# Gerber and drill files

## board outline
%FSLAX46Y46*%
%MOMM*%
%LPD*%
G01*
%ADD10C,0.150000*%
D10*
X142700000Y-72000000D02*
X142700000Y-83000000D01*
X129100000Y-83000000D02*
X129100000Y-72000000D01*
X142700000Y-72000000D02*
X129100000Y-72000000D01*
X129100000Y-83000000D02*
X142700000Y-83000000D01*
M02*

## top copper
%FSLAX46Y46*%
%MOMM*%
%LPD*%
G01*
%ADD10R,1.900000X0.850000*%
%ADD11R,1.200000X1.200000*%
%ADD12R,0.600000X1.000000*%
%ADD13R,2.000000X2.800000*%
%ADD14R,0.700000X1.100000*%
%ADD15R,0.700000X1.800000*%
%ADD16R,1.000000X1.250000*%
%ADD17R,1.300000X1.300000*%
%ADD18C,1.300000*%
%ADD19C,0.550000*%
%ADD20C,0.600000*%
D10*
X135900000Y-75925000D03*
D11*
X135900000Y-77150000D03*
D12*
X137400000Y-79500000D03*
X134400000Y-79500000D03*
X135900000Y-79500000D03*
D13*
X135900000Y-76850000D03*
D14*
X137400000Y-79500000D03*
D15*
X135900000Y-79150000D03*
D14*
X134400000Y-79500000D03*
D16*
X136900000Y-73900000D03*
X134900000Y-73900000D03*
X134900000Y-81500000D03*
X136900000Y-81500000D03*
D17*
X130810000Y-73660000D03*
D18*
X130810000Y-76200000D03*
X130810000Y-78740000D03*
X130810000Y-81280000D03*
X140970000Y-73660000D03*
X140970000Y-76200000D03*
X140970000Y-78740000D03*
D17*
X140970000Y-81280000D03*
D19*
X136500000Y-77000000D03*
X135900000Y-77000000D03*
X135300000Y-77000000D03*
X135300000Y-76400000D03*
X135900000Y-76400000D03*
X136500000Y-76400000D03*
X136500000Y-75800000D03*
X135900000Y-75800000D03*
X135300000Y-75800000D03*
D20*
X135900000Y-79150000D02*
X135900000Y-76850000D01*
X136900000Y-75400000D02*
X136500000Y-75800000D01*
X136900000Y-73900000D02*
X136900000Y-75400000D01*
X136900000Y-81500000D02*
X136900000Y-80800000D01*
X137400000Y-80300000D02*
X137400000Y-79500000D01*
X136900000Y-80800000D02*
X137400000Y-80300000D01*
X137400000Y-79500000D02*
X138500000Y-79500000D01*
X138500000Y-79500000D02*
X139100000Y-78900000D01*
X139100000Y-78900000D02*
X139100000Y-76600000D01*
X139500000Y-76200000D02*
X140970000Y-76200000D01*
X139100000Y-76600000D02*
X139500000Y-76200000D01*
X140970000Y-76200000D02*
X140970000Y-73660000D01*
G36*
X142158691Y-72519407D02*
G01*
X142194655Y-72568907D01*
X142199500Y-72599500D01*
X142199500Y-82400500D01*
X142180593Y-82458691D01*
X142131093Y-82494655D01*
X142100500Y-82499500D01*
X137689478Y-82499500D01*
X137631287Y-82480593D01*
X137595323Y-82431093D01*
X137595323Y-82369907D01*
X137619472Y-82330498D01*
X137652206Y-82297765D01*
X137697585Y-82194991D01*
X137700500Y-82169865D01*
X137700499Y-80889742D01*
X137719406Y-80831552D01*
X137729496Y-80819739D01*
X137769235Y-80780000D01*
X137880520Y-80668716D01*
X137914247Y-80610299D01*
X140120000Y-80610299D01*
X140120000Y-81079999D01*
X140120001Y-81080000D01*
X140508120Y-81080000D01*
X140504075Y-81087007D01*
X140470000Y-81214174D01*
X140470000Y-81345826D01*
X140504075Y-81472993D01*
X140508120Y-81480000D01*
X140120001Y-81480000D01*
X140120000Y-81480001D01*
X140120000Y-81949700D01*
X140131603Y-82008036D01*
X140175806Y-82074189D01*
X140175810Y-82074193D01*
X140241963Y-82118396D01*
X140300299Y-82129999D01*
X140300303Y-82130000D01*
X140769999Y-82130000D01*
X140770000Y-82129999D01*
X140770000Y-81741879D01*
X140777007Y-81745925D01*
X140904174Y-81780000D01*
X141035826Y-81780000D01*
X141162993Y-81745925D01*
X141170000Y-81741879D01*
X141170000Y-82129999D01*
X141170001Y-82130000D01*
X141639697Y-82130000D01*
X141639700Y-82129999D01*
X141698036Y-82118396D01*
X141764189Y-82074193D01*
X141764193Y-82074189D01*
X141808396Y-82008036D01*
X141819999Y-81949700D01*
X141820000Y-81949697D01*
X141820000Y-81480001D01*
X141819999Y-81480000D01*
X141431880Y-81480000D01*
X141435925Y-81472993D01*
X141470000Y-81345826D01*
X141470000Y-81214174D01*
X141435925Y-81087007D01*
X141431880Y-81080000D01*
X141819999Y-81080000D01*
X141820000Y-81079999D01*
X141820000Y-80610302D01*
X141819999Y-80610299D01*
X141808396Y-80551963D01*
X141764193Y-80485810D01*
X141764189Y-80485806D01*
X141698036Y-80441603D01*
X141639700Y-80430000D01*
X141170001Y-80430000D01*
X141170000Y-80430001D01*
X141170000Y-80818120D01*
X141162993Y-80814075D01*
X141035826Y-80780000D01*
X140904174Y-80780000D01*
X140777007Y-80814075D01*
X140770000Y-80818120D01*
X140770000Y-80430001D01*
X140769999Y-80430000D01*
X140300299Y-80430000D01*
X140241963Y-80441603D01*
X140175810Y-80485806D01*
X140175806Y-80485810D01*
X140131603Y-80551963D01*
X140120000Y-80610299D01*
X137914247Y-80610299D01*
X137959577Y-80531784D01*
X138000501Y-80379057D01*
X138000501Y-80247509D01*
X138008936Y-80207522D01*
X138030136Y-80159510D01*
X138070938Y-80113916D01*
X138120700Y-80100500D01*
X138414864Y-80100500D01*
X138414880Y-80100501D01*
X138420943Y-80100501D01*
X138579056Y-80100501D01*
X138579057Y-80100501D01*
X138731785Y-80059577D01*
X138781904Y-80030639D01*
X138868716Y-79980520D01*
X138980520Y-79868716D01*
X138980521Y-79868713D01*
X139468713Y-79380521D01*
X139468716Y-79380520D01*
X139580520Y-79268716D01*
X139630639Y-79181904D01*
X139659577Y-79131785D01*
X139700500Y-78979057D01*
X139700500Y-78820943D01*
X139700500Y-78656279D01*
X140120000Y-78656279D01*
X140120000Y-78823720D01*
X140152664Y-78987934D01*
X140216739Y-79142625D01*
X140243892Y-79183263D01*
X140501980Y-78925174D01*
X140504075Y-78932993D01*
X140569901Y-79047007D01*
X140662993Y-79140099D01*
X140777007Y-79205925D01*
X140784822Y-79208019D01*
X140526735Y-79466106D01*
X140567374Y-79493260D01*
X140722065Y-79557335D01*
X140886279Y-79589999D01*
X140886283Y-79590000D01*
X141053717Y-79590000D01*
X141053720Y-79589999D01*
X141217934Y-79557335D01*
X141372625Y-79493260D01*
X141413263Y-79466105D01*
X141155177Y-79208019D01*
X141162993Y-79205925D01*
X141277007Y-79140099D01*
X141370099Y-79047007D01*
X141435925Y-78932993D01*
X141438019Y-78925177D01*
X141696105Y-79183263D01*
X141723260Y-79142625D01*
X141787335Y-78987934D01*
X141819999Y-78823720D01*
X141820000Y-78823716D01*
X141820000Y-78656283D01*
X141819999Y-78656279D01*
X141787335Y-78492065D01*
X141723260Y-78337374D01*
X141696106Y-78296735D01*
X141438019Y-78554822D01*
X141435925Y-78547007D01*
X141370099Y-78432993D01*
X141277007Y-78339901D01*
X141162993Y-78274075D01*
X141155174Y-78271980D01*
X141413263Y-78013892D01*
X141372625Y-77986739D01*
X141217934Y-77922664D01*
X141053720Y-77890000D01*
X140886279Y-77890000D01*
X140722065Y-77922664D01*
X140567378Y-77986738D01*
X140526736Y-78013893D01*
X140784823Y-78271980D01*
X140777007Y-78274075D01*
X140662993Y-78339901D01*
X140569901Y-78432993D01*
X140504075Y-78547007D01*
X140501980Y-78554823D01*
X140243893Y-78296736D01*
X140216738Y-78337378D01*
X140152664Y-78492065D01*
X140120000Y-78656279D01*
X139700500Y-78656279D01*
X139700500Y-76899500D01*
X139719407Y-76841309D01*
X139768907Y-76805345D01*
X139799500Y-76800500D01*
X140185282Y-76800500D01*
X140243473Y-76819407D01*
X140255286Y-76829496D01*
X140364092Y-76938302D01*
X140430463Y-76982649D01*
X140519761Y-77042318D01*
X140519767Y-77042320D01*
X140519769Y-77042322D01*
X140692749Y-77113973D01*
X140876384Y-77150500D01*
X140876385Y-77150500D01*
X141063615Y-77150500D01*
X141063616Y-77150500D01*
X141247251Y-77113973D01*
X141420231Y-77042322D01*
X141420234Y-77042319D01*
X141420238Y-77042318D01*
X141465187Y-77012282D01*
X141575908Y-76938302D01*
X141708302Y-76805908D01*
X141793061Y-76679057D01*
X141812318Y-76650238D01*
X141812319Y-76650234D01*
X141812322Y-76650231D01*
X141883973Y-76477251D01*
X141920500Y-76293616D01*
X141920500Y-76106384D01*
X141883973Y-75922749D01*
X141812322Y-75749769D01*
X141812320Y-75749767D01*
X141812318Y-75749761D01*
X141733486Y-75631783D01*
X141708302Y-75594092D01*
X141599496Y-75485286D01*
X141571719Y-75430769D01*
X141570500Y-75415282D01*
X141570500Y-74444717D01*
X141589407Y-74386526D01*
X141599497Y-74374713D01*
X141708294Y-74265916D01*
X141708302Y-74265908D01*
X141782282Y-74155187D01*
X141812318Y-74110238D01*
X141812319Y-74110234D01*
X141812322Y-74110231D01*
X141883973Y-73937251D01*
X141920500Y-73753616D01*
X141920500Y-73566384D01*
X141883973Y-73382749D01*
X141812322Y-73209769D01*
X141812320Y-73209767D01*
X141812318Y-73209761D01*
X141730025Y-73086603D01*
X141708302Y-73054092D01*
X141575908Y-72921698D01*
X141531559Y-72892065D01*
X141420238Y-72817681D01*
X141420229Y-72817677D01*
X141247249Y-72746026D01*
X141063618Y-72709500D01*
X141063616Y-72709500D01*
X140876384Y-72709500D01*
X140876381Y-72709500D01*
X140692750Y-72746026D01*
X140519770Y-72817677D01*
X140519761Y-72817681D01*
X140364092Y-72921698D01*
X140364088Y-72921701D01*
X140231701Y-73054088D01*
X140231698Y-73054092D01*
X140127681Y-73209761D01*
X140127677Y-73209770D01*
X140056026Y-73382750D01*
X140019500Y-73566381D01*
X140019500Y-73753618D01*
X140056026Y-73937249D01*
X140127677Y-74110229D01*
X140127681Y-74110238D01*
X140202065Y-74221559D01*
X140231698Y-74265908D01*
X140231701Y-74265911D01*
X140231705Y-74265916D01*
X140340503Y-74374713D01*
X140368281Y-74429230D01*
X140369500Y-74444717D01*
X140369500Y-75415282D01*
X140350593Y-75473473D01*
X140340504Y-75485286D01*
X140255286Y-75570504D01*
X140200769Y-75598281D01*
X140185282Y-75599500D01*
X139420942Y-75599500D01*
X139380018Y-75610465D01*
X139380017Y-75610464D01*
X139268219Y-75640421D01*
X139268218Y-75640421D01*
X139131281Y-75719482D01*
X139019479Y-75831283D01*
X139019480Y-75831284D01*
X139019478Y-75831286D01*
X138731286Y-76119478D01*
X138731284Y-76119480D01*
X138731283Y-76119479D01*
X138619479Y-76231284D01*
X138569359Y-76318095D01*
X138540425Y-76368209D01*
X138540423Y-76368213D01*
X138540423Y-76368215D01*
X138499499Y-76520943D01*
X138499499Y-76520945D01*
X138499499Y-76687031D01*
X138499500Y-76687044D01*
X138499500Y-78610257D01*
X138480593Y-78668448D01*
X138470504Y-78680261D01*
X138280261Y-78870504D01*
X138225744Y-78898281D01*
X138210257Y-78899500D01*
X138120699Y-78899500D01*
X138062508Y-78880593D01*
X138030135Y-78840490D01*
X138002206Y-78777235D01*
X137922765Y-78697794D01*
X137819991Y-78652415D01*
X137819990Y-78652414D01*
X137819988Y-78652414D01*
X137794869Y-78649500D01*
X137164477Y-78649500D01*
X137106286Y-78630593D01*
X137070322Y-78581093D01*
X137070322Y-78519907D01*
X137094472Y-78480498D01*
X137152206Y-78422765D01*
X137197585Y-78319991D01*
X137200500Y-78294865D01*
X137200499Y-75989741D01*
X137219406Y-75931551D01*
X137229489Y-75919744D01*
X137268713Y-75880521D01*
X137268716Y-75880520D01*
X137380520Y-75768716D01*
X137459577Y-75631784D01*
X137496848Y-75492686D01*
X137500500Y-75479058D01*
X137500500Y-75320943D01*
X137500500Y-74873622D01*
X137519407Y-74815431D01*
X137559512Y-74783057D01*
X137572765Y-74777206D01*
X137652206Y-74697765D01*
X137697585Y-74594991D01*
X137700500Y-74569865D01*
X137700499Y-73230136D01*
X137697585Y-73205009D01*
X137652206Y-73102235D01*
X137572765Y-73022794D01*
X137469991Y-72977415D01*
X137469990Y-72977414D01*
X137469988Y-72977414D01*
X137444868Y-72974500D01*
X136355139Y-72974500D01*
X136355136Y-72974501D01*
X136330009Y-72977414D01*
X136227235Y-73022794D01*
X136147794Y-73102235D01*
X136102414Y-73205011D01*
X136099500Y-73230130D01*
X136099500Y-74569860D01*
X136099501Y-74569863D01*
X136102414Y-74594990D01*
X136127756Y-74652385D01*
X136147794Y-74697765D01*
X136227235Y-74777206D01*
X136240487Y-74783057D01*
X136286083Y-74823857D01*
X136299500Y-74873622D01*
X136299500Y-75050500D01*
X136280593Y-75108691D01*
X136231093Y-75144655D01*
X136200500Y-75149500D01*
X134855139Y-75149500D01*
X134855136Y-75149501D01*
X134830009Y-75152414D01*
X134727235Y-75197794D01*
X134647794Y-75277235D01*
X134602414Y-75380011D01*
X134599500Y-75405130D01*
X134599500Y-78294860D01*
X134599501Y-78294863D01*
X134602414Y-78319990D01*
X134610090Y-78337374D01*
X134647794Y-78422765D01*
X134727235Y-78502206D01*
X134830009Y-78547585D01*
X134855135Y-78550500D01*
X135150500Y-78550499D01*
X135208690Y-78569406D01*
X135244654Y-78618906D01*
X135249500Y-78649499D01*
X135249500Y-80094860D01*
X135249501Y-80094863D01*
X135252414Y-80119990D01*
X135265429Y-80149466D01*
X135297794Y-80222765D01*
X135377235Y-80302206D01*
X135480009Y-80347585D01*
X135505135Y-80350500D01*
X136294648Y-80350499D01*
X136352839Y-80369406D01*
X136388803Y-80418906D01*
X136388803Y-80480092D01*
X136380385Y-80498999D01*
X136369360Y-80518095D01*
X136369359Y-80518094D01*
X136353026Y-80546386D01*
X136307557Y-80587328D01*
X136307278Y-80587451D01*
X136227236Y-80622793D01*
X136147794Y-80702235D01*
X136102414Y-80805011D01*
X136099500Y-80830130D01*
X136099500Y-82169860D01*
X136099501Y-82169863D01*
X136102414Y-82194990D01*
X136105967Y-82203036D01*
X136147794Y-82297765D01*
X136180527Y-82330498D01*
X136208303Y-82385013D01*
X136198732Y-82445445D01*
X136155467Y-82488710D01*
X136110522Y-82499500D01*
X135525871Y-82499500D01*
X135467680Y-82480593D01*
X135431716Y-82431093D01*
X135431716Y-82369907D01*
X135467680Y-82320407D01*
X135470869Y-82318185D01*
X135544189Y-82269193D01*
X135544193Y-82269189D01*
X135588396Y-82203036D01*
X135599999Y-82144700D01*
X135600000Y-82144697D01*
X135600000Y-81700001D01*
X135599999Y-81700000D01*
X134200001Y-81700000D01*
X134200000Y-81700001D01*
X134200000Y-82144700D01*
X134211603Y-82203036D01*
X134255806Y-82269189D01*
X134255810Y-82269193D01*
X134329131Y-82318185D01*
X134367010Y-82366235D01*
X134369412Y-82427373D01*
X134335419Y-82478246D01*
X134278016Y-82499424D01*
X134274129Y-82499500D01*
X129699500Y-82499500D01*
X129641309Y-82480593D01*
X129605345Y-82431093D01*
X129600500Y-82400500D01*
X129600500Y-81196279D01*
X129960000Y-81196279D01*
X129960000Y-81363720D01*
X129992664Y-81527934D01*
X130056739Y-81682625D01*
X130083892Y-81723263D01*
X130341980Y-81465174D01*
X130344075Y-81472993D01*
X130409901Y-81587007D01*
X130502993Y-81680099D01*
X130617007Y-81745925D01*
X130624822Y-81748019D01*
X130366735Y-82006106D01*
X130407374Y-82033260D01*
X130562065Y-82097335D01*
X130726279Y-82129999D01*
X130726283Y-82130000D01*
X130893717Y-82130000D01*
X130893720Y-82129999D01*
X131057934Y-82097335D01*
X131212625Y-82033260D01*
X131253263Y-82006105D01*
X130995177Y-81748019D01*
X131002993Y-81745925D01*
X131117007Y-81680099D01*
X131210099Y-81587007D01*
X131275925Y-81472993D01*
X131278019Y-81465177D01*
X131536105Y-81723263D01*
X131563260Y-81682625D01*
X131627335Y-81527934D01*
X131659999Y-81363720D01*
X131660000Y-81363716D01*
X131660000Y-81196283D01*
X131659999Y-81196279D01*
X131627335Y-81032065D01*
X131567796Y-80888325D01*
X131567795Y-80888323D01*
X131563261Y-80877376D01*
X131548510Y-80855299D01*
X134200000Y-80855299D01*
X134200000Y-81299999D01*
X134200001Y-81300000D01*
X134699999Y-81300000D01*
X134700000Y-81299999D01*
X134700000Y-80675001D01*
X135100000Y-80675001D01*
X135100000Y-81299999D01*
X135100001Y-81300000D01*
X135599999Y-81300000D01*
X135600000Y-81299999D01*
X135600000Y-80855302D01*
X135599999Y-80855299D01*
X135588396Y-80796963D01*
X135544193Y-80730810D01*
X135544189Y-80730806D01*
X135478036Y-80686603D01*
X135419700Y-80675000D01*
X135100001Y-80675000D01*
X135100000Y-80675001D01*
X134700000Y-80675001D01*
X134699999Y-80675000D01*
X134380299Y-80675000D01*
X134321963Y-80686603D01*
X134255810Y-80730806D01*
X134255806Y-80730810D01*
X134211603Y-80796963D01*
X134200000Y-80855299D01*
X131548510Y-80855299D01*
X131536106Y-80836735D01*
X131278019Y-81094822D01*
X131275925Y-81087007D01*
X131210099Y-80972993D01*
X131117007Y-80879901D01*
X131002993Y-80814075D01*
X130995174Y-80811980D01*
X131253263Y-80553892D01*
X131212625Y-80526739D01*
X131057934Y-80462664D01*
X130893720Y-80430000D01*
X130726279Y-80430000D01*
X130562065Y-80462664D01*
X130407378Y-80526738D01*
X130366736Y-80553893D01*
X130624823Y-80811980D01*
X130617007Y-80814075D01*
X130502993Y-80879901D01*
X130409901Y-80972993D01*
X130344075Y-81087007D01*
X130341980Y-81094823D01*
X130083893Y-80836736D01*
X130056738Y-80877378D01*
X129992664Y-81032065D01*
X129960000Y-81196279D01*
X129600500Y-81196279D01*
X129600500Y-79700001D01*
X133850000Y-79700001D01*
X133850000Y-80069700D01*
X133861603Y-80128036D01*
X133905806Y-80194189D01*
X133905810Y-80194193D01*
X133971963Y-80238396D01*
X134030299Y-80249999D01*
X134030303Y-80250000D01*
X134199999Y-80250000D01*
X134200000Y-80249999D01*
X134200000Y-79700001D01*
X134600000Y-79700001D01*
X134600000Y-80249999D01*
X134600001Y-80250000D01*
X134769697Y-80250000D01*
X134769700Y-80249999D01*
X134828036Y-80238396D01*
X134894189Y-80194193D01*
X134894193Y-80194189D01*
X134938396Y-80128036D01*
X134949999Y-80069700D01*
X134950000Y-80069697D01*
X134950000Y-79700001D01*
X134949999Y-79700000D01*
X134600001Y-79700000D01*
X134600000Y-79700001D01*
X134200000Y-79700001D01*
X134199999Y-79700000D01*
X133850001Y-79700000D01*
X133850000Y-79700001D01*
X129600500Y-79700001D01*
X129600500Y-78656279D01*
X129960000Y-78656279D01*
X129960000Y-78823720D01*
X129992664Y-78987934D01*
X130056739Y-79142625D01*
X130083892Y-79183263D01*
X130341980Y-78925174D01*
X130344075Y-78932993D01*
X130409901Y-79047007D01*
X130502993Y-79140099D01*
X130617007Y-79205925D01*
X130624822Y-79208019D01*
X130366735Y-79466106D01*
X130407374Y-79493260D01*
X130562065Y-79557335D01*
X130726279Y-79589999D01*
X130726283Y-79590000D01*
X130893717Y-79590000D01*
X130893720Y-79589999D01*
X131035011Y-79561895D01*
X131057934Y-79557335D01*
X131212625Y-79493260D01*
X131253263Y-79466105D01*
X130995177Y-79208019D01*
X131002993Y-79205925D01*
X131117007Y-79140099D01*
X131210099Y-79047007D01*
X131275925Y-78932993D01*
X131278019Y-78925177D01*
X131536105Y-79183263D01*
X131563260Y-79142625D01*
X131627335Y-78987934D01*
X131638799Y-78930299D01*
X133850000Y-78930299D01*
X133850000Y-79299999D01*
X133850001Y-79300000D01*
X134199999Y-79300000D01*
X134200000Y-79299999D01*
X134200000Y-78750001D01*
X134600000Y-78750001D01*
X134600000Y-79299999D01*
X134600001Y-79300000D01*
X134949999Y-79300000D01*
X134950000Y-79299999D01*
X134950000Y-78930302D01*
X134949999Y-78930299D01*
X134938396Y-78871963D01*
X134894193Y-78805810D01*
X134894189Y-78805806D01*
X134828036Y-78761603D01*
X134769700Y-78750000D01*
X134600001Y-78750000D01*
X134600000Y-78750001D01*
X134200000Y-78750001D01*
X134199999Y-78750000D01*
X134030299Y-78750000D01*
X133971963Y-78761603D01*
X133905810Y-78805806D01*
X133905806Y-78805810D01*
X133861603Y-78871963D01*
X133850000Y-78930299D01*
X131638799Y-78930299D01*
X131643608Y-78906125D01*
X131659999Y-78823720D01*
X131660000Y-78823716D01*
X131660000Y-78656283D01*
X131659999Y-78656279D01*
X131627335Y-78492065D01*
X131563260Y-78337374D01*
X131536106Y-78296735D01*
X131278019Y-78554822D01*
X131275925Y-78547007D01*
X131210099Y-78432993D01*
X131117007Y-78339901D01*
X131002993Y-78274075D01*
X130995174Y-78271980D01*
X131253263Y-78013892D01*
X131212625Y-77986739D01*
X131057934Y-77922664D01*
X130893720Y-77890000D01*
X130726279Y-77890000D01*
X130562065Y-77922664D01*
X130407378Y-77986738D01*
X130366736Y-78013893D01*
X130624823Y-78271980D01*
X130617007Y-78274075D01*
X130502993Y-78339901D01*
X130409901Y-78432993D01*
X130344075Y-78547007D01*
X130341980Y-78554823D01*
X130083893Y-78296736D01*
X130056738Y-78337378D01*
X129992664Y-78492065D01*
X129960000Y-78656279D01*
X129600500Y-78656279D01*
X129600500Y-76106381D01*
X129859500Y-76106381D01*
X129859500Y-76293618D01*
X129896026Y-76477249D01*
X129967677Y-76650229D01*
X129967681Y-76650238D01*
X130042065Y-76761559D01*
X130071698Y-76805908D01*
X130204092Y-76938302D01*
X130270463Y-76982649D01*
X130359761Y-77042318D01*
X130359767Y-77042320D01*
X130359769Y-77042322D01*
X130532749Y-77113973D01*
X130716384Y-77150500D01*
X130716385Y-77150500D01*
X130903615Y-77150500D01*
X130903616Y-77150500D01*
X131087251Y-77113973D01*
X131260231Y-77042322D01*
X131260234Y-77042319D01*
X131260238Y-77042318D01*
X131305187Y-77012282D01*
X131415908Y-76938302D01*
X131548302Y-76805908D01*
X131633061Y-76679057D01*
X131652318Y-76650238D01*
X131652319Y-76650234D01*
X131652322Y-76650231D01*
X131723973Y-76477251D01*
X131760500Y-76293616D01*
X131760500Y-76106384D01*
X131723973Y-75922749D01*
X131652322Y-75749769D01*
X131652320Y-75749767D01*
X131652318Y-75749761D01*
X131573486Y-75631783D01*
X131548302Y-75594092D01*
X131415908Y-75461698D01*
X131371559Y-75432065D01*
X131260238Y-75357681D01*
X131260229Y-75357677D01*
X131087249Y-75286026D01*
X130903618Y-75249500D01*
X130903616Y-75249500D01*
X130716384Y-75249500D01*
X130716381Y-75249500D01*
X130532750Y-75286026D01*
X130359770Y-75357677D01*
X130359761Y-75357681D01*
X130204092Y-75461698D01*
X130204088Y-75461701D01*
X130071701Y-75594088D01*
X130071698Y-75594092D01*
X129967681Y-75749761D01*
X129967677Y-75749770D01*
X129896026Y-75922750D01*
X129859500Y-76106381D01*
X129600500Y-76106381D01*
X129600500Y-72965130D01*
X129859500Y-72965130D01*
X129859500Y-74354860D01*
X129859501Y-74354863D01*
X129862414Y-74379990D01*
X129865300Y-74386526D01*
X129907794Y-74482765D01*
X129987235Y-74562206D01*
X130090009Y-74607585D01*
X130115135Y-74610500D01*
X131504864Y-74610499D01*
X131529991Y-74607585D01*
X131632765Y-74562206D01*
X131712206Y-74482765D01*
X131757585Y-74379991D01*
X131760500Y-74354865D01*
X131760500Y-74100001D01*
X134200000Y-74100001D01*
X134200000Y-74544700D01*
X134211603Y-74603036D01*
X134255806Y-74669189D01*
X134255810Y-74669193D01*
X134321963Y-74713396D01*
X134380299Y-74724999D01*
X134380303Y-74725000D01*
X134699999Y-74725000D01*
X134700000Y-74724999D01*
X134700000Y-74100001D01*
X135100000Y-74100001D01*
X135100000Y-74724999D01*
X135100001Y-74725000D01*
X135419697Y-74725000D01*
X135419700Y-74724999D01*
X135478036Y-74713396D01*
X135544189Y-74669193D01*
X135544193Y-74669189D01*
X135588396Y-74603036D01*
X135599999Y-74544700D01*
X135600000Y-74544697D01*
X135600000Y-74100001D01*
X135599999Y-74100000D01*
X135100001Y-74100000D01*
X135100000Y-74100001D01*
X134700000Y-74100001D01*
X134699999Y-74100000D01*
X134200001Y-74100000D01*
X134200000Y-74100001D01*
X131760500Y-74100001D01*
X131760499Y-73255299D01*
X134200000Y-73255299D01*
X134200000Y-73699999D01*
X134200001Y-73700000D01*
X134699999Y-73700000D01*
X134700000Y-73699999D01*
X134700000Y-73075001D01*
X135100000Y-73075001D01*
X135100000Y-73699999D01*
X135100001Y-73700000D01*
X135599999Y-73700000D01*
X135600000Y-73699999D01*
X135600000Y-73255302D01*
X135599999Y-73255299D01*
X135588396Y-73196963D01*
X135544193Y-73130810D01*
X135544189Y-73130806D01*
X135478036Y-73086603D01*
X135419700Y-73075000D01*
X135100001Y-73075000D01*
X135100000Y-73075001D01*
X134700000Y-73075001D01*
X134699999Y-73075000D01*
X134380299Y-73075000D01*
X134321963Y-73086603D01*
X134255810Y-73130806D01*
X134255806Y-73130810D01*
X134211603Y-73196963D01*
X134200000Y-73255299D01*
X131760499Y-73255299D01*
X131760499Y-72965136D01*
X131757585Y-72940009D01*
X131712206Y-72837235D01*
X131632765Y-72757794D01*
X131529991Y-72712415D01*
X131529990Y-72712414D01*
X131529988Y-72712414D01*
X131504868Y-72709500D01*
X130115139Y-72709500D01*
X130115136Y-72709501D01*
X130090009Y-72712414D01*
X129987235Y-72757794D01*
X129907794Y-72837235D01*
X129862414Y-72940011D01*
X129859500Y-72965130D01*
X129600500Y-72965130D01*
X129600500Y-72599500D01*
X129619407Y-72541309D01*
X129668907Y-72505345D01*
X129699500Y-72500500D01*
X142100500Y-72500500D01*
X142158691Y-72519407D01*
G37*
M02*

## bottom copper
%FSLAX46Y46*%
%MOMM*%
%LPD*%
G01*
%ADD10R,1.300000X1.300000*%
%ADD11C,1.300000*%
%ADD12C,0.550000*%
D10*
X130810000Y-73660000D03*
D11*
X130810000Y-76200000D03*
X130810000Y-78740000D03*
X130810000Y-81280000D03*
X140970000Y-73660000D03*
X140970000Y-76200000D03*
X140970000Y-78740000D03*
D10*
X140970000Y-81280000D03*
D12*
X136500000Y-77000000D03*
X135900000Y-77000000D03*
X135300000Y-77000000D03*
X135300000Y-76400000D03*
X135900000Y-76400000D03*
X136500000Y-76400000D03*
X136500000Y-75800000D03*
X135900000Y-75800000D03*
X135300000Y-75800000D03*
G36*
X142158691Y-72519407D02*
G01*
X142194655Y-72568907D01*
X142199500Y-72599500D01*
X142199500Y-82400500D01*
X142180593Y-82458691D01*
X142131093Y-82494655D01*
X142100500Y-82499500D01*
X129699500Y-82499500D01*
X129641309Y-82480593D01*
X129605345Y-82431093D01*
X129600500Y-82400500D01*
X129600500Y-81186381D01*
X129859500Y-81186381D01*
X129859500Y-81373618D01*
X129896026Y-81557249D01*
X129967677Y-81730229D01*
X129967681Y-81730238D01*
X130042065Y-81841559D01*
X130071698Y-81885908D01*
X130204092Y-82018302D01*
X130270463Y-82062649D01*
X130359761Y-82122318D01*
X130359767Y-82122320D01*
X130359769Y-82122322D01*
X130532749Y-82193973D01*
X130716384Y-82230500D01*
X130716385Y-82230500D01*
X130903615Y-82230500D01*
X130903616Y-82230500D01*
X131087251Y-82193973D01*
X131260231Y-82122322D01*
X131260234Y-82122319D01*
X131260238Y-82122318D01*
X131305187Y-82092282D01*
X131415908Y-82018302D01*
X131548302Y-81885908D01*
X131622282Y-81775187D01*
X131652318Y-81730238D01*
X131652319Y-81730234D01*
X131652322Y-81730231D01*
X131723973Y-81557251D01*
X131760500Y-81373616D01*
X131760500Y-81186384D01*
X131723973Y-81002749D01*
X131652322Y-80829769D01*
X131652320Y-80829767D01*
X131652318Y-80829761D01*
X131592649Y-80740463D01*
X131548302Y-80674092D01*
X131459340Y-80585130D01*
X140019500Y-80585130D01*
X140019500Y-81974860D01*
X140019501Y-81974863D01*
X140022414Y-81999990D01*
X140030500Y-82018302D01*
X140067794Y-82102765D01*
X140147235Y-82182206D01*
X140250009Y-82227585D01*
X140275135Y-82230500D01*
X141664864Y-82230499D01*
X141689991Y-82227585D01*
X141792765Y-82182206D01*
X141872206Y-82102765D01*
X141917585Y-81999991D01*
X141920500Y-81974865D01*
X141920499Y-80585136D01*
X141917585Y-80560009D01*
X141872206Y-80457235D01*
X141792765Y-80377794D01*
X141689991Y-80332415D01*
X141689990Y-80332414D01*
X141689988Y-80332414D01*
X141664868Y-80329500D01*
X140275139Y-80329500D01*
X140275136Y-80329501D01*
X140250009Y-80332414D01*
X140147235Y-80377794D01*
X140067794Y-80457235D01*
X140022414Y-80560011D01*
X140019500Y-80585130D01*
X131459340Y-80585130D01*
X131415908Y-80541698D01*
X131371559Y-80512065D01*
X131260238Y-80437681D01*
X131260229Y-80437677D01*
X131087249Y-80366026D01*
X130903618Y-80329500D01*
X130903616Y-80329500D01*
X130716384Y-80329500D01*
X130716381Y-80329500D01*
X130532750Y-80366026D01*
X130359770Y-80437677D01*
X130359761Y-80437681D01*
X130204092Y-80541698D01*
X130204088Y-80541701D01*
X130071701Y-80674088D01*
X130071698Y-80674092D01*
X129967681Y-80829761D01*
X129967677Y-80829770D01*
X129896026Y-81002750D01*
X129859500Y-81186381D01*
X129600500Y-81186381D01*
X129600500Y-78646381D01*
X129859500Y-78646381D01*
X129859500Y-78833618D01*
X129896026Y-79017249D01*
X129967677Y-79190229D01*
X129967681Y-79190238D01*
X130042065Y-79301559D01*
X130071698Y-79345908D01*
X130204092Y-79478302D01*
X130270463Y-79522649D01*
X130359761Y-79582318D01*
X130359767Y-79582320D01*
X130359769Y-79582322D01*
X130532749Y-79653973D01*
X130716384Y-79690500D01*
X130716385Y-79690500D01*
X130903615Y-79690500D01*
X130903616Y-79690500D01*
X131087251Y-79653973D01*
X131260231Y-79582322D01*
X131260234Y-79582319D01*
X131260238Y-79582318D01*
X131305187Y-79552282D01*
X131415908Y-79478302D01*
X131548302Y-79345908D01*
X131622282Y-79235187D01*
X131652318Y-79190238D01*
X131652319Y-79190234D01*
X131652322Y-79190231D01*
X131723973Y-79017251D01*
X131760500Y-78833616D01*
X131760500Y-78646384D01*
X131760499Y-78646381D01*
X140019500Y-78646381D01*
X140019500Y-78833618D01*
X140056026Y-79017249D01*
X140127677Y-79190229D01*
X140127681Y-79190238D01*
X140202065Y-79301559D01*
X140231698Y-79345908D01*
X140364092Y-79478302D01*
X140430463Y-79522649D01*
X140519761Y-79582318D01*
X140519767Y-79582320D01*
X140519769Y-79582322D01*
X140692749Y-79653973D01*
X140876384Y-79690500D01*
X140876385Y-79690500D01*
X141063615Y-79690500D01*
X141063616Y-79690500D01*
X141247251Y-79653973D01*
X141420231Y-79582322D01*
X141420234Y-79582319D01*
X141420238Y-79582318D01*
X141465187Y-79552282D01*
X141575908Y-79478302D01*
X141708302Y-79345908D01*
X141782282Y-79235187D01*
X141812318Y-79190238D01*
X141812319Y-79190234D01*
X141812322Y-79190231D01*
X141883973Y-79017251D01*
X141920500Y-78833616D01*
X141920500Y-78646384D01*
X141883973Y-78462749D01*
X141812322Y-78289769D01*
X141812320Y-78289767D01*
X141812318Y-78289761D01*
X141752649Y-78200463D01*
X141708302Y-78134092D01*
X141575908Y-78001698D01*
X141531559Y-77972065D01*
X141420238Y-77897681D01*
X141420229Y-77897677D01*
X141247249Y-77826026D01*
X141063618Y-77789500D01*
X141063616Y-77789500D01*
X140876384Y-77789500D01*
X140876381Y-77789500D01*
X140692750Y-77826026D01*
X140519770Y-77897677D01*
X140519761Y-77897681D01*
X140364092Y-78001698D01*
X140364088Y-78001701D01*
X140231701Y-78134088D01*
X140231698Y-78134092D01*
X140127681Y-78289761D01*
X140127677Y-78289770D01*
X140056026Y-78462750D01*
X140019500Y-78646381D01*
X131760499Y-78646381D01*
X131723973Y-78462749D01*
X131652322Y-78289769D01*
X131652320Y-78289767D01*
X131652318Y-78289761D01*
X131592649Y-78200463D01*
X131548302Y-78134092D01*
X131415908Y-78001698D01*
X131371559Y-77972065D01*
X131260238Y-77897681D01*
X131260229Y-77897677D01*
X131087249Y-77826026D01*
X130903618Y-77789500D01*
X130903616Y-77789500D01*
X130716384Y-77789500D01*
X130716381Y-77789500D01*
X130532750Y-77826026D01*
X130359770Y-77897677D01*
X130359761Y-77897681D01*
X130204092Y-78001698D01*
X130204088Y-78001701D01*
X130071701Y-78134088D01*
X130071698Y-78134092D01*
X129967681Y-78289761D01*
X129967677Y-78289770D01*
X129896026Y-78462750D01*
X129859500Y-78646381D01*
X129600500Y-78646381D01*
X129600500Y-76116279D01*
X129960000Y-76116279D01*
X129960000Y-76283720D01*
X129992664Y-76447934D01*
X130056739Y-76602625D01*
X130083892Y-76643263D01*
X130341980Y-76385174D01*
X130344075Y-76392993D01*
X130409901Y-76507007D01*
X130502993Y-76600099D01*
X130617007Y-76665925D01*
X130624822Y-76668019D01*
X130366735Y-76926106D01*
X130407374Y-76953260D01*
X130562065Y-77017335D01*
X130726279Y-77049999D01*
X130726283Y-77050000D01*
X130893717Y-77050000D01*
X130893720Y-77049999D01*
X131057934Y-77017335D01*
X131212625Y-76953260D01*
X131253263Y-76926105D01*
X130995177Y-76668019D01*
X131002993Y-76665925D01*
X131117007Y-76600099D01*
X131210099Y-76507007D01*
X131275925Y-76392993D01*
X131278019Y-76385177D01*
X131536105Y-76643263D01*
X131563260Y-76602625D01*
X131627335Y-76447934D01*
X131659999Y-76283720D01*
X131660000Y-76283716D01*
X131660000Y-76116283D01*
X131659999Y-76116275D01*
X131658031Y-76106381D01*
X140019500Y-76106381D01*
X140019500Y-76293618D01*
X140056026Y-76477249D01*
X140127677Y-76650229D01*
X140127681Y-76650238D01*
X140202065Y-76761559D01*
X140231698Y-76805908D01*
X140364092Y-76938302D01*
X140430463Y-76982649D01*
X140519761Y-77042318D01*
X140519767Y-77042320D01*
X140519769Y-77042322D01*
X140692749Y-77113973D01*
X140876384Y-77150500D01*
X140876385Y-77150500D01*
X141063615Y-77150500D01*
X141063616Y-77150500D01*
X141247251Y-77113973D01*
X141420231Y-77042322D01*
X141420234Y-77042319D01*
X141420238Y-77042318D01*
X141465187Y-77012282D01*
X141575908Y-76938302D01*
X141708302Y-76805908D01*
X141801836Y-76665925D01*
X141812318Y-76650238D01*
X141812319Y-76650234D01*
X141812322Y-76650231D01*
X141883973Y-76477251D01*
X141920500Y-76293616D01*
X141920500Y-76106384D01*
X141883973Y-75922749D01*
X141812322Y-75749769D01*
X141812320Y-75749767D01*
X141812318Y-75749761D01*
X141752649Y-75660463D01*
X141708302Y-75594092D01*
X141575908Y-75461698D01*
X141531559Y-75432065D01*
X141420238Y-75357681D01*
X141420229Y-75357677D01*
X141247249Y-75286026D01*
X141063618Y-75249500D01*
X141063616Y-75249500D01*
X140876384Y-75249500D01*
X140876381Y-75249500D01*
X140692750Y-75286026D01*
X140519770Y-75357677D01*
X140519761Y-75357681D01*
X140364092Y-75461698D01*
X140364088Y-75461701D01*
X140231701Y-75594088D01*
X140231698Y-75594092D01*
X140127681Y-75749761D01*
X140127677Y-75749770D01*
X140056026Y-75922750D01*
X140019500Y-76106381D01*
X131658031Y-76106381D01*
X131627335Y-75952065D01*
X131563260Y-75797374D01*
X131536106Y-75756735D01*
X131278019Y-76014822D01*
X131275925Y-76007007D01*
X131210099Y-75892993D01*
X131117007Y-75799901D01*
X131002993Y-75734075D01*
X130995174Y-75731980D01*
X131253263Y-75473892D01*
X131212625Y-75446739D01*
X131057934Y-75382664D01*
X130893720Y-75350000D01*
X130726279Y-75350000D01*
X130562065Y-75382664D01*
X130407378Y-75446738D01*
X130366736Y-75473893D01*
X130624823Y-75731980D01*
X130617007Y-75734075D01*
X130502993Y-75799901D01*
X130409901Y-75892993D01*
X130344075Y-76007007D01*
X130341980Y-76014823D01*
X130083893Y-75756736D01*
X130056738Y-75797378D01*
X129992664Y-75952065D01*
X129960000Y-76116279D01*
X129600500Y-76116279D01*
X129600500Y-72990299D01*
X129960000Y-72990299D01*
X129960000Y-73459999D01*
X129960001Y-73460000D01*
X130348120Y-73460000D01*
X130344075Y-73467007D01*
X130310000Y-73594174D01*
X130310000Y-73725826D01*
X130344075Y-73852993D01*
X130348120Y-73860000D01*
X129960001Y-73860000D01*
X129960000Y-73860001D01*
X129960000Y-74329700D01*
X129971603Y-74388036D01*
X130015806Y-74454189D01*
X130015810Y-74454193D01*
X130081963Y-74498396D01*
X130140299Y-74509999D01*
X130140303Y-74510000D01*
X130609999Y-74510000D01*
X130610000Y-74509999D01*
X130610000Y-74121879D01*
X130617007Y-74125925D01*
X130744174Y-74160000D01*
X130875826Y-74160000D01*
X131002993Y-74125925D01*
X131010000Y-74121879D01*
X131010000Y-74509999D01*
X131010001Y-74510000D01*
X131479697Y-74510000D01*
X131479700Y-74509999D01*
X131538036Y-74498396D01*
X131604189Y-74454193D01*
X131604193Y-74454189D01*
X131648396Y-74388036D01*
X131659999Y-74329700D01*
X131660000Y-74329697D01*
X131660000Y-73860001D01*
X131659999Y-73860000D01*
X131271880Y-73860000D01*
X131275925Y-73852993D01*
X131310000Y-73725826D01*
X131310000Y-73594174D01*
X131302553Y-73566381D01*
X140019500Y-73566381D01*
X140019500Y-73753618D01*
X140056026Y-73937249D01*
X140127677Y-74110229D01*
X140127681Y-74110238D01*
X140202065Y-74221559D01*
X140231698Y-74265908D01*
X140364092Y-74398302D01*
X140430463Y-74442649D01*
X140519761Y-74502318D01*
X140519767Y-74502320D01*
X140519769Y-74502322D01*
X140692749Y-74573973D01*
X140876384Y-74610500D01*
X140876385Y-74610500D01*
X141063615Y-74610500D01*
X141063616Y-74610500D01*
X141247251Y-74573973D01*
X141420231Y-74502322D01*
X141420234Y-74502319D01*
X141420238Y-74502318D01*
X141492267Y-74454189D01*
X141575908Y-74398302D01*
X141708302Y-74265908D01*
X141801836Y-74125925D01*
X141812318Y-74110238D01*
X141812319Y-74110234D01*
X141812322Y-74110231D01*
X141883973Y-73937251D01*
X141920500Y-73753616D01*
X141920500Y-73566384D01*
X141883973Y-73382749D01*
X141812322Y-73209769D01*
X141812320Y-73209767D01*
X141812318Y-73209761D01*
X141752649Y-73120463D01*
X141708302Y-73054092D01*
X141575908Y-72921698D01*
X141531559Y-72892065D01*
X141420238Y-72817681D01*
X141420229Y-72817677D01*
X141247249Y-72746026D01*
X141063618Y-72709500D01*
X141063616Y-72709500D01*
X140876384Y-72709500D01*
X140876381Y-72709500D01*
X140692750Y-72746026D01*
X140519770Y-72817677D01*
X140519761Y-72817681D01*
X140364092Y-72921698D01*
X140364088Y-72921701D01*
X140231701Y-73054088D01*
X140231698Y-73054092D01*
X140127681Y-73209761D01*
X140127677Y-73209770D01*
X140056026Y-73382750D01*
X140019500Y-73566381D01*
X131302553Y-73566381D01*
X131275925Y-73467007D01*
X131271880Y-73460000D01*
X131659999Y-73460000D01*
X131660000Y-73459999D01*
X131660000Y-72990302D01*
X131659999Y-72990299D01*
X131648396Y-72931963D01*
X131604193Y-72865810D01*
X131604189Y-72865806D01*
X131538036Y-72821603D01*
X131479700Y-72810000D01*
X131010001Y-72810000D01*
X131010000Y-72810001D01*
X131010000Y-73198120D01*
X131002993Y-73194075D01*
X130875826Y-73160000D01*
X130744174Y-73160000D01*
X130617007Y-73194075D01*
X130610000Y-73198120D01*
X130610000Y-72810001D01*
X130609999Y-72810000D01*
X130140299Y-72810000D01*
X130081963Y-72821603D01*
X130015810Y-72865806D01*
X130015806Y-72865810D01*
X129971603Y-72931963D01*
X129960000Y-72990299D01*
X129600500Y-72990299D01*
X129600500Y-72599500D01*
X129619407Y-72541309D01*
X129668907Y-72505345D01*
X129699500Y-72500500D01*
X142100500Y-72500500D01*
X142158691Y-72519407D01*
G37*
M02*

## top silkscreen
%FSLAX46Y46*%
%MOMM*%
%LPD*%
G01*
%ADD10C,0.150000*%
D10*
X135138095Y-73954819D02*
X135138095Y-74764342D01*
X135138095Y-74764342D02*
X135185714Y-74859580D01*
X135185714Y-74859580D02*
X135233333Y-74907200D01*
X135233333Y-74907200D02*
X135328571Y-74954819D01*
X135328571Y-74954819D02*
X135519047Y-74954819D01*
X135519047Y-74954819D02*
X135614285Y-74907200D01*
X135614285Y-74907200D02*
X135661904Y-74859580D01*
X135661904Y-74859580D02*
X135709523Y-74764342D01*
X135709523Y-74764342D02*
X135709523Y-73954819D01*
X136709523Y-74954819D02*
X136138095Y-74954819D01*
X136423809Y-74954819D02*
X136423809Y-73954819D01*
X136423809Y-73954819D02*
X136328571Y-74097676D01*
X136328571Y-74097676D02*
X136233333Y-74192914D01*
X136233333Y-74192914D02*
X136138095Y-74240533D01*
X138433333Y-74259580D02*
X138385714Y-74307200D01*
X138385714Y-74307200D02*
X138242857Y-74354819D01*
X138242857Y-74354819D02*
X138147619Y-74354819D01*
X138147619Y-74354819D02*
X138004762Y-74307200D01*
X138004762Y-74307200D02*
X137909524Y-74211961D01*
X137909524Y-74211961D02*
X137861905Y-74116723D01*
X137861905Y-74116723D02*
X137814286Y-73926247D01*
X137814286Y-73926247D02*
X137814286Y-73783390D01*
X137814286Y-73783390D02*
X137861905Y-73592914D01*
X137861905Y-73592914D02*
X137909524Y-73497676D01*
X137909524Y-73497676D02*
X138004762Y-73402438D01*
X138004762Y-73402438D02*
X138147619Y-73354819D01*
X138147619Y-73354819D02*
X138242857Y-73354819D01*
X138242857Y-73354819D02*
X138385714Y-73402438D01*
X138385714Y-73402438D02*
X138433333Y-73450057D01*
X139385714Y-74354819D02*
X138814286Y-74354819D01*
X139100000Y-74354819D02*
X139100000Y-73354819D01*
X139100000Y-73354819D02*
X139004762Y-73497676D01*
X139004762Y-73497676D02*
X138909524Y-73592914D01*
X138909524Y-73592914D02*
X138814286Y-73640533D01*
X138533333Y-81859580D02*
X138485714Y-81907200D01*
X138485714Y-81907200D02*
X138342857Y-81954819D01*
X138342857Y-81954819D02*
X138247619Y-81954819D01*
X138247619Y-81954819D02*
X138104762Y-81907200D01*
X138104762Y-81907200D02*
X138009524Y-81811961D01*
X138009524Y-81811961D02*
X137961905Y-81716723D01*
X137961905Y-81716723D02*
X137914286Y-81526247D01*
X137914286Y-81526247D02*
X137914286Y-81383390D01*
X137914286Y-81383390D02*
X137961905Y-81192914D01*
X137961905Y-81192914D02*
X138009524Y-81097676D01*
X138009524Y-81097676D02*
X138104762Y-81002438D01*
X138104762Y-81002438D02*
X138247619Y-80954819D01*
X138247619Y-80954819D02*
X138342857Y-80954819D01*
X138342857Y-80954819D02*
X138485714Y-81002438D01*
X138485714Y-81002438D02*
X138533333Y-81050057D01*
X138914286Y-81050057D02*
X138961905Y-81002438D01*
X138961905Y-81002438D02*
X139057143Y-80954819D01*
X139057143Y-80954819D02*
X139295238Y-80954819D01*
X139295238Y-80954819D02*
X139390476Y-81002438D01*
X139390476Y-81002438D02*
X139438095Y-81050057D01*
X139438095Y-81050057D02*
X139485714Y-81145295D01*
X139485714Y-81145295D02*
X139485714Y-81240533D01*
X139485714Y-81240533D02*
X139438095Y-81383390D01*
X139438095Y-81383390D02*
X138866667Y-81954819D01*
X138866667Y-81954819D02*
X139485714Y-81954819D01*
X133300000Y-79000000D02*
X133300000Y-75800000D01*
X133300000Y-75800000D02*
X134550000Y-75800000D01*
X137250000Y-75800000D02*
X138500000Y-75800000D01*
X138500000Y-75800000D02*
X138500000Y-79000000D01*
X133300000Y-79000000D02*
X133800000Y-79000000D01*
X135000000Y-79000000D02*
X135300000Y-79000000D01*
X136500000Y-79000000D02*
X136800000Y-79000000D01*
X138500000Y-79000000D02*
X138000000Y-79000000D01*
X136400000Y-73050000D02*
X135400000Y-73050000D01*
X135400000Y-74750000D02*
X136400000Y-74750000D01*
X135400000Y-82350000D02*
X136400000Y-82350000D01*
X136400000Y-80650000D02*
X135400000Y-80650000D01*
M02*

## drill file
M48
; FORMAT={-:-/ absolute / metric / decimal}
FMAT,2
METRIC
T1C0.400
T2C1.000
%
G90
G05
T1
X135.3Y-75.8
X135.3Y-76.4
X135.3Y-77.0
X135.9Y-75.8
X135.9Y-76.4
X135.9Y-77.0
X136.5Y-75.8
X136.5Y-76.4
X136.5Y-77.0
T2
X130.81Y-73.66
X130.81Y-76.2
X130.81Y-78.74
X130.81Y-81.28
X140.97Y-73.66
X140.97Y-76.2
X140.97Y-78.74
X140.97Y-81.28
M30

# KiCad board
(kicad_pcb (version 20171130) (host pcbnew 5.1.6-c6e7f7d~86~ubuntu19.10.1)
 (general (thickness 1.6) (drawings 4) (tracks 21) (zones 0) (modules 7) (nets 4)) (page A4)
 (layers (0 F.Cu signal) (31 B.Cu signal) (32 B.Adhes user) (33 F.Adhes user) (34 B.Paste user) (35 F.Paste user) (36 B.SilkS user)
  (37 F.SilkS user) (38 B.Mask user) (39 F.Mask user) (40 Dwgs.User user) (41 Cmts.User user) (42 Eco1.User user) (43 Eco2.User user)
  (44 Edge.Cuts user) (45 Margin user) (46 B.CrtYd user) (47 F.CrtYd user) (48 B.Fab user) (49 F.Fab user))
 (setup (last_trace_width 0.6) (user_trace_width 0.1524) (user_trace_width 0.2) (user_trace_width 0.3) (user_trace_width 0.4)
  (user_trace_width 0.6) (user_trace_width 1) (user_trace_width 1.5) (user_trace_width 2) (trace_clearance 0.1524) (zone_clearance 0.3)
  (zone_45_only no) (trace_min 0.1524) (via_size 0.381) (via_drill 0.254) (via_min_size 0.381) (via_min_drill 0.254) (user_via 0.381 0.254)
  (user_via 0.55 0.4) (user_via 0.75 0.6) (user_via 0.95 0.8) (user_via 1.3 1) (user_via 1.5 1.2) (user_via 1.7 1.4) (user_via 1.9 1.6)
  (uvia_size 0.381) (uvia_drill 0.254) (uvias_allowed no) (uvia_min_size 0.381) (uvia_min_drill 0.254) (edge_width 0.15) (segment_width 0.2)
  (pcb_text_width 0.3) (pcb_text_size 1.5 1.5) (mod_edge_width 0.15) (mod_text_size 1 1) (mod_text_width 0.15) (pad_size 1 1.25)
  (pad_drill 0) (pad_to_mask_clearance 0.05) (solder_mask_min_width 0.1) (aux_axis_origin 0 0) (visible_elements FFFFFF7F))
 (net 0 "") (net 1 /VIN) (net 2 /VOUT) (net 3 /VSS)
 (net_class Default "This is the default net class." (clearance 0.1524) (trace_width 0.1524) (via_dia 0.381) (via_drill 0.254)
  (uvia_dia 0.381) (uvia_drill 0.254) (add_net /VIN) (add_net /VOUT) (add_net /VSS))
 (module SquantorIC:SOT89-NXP (layer F.Cu) (at 135.9 77.75)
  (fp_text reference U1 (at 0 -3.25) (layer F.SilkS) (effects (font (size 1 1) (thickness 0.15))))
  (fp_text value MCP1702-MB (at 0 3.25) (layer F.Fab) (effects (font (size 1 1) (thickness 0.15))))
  (fp_line (start -2.6 1.25) (end -2.6 -1.95) (layer F.SilkS) (width 0.15))
  (fp_line (start -2.6 -1.95) (end -1.35 -1.95) (layer F.SilkS) (width 0.15))
  (fp_line (start 1.35 -1.95) (end 2.6 -1.95) (layer F.SilkS) (width 0.15))
  (fp_line (start 2.6 -1.95) (end 2.6 1.25) (layer F.SilkS) (width 0.15))
  (fp_line (start -2.6 1.25) (end -2.1 1.25) (layer F.SilkS) (width 0.15))
  (fp_line (start -0.9 1.25) (end -0.6 1.25) (layer F.SilkS) (width 0.15))
  (fp_line (start 0.6 1.25) (end 0.9 1.25) (layer F.SilkS) (width 0.15))
  (fp_line (start 2.6 1.25) (end 2.1 1.25) (layer F.SilkS) (width 0.15))
  (pad 2 smd rect (at 0 -1.825) (size 1.9 0.85) (layers F.Cu F.Paste) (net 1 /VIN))
  (pad 2 smd rect (at 0 -0.6) (size 1.2 1.2) (layers F.Cu F.Paste) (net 1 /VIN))
  (pad 3 smd rect (at 1.5 1.75) (size 0.6 1) (layers F.Cu F.Paste) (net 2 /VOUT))
  (pad 1 smd rect (at -1.5 1.75) (size 0.6 1) (layers F.Cu F.Paste) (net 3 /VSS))
  (pad 2 smd rect (at 0 1.75) (size 0.6 1) (layers F.Cu F.Paste) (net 1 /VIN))
  (pad 2 smd rect (at 0 -0.9) (size 2 2.8) (layers F.Cu F.Mask) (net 1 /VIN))
  (pad 3 smd rect (at 1.5 1.75) (size 0.7 1.1) (layers F.Cu F.Mask) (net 2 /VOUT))
  (pad 2 smd rect (at 0 1.4) (size 0.7 1.8) (layers F.Cu F.Mask) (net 1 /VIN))
  (pad 1 smd rect (at -1.5 1.75) (size 0.7 1.1) (layers F.Cu F.Mask) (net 3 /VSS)))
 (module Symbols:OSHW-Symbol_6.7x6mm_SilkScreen (layer B.Cu) (at 135.9 75.3 180)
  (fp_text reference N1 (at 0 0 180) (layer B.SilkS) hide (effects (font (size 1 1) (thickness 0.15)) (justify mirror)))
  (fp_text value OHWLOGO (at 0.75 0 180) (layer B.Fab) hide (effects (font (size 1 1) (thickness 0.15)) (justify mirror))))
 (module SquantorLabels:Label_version (layer B.Cu) (at 135.3 80.01 90)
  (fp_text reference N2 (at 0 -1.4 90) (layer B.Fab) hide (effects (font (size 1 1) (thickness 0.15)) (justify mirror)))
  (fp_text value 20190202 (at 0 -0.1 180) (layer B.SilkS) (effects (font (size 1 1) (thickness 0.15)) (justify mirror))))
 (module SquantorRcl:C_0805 (layer F.Cu) (at 135.9 73.9 180)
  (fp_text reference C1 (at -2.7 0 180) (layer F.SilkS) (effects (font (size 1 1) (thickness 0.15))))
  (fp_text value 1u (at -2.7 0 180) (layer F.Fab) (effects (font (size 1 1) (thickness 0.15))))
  (fp_line (start -0.5 0.85) (end 0.5 0.85) (layer F.SilkS) (width 0.15))
  (fp_line (start 0.5 -0.85) (end -0.5 -0.85) (layer F.SilkS) (width 0.15))
  (pad 1 smd rect (at -1 0 180) (size 1 1.25) (layers F.Cu F.Paste F.Mask) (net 1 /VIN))
  (pad 2 smd rect (at 1 0 180) (size 1 1.25) (layers F.Cu F.Paste F.Mask) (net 3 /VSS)))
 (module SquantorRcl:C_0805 (layer F.Cu) (at 135.9 81.5 180)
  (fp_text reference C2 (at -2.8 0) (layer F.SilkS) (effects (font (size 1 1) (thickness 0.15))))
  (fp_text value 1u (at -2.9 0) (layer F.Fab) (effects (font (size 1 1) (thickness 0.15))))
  (fp_line (start 0.5 -0.85) (end -0.5 -0.85) (layer F.SilkS) (width 0.15))
  (fp_line (start -0.5 0.85) (end 0.5 0.85) (layer F.SilkS) (width 0.15))
  (pad 2 smd rect (at 1 0 180) (size 1 1.25) (layers F.Cu F.Paste F.Mask) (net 3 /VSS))
  (pad 1 smd rect (at -1 0 180) (size 1 1.25) (layers F.Cu F.Paste F.Mask) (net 2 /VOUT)))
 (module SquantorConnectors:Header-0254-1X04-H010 (layer B.Cu) (at 130.81 77.47 270)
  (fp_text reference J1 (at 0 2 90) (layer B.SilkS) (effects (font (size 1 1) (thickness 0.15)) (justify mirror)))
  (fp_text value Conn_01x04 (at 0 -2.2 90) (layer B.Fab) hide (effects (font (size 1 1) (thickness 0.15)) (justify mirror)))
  (pad 1 thru_hole rect (at -3.81 0 90) (size 1.3 1.3) (drill 1) (layers *.Cu *.Mask) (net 1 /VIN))
  (pad 2 thru_hole circle (at -1.27 0 90) (size 1.3 1.3) (drill 1) (layers *.Cu *.Mask) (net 1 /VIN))
  (pad 3 thru_hole circle (at 1.27 0 90) (size 1.3 1.3) (drill 1) (layers *.Cu *.Mask) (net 3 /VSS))
  (pad 4 thru_hole circle (at 3.81 0 90) (size 1.3 1.3) (drill 1) (layers *.Cu *.Mask) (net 3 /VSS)))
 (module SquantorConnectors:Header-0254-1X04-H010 (layer B.Cu) (at 140.97 77.47 90)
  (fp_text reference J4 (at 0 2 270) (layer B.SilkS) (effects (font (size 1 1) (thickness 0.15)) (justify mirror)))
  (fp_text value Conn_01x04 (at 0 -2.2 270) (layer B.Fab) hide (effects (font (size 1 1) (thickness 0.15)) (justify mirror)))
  (pad 4 thru_hole circle (at 3.81 0 270) (size 1.3 1.3) (drill 1) (layers *.Cu *.Mask) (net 2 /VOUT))
  (pad 3 thru_hole circle (at 1.27 0 270) (size 1.3 1.3) (drill 1) (layers *.Cu *.Mask) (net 2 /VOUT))
  (pad 2 thru_hole circle (at -1.27 0 270) (size 1.3 1.3) (drill 1) (layers *.Cu *.Mask) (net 3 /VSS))
  (pad 1 thru_hole rect (at -3.81 0 270) (size 1.3 1.3) (drill 1) (layers *.Cu *.Mask) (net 3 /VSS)))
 (gr_line (start 142.7 72) (end 142.7 83) (layer Edge.Cuts) (width 0.15))
 (gr_line (start 129.1 83) (end 129.1 72) (layer Edge.Cuts) (width 0.15))
 (gr_line (start 142.7 72) (end 129.1 72) (layer Edge.Cuts) (width 0.15))
 (gr_line (start 129.1 83) (end 142.7 83) (layer Edge.Cuts) (width 0.15))
 (via (at 136.5 77) (size 0.55) (drill 0.4) (layers F.Cu B.Cu) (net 1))
 (via (at 135.9 77) (size 0.55) (drill 0.4) (layers F.Cu B.Cu) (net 1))
 (via (at 135.3 77) (size 0.55) (drill 0.4) (layers F.Cu B.Cu) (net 1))
 (via (at 135.3 76.4) (size 0.55) (drill 0.4) (layers F.Cu B.Cu) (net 1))
 (via (at 135.9 76.4) (size 0.55) (drill 0.4) (layers F.Cu B.Cu) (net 1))
 (via (at 136.5 76.4) (size 0.55) (drill 0.4) (layers F.Cu B.Cu) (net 1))
 (via (at 136.5 75.8) (size 0.55) (drill 0.4) (layers F.Cu B.Cu) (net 1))
 (via (at 135.9 75.8) (size 0.55) (drill 0.4) (layers F.Cu B.Cu) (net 1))
 (via (at 135.3 75.8) (size 0.55) (drill 0.4) (layers F.Cu B.Cu) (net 1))
 (segment (start 135.9 79.15) (end 135.9 76.85) (width 0.6) (layer F.Cu) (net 1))
 (segment (start 136.9 75.4) (end 136.5 75.8) (width 0.6) (layer F.Cu) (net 1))
 (segment (start 136.9 73.9) (end 136.9 75.4) (width 0.6) (layer F.Cu) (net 1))
 (segment (start 136.9 81.5) (end 136.9 80.8) (width 0.6) (layer F.Cu) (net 2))
 (segment (start 137.4 80.3) (end 137.4 79.5) (width 0.6) (layer F.Cu) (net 2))
 (segment (start 136.9 80.8) (end 137.4 80.3) (width 0.6) (layer F.Cu) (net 2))
 (segment (start 137.4 79.5) (end 138.5 79.5) (width 0.6) (layer F.Cu) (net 2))
 (segment (start 138.5 79.5) (end 139.1 78.9) (width 0.6) (layer F.Cu) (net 2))
 (segment (start 139.1 78.9) (end 139.1 76.6) (width 0.6) (layer F.Cu) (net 2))
 (segment (start 139.5 76.2) (end 140.97 76.2) (width 0.6) (layer F.Cu) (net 2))
 (segment (start 139.1 76.6) (end 139.5 76.2) (width 0.6) (layer F.Cu) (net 2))
 (segment (start 140.97 76.2) (end 140.97 73.66) (width 0.6) (layer F.Cu) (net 2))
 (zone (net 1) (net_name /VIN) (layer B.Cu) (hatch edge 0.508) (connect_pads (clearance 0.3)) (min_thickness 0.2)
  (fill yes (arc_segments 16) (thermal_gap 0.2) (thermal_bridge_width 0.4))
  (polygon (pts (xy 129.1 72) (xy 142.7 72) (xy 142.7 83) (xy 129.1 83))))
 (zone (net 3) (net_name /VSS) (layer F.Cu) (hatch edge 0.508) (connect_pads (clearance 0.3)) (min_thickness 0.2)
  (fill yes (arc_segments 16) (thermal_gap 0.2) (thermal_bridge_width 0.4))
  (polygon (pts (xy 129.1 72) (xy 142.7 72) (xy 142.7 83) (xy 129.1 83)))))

